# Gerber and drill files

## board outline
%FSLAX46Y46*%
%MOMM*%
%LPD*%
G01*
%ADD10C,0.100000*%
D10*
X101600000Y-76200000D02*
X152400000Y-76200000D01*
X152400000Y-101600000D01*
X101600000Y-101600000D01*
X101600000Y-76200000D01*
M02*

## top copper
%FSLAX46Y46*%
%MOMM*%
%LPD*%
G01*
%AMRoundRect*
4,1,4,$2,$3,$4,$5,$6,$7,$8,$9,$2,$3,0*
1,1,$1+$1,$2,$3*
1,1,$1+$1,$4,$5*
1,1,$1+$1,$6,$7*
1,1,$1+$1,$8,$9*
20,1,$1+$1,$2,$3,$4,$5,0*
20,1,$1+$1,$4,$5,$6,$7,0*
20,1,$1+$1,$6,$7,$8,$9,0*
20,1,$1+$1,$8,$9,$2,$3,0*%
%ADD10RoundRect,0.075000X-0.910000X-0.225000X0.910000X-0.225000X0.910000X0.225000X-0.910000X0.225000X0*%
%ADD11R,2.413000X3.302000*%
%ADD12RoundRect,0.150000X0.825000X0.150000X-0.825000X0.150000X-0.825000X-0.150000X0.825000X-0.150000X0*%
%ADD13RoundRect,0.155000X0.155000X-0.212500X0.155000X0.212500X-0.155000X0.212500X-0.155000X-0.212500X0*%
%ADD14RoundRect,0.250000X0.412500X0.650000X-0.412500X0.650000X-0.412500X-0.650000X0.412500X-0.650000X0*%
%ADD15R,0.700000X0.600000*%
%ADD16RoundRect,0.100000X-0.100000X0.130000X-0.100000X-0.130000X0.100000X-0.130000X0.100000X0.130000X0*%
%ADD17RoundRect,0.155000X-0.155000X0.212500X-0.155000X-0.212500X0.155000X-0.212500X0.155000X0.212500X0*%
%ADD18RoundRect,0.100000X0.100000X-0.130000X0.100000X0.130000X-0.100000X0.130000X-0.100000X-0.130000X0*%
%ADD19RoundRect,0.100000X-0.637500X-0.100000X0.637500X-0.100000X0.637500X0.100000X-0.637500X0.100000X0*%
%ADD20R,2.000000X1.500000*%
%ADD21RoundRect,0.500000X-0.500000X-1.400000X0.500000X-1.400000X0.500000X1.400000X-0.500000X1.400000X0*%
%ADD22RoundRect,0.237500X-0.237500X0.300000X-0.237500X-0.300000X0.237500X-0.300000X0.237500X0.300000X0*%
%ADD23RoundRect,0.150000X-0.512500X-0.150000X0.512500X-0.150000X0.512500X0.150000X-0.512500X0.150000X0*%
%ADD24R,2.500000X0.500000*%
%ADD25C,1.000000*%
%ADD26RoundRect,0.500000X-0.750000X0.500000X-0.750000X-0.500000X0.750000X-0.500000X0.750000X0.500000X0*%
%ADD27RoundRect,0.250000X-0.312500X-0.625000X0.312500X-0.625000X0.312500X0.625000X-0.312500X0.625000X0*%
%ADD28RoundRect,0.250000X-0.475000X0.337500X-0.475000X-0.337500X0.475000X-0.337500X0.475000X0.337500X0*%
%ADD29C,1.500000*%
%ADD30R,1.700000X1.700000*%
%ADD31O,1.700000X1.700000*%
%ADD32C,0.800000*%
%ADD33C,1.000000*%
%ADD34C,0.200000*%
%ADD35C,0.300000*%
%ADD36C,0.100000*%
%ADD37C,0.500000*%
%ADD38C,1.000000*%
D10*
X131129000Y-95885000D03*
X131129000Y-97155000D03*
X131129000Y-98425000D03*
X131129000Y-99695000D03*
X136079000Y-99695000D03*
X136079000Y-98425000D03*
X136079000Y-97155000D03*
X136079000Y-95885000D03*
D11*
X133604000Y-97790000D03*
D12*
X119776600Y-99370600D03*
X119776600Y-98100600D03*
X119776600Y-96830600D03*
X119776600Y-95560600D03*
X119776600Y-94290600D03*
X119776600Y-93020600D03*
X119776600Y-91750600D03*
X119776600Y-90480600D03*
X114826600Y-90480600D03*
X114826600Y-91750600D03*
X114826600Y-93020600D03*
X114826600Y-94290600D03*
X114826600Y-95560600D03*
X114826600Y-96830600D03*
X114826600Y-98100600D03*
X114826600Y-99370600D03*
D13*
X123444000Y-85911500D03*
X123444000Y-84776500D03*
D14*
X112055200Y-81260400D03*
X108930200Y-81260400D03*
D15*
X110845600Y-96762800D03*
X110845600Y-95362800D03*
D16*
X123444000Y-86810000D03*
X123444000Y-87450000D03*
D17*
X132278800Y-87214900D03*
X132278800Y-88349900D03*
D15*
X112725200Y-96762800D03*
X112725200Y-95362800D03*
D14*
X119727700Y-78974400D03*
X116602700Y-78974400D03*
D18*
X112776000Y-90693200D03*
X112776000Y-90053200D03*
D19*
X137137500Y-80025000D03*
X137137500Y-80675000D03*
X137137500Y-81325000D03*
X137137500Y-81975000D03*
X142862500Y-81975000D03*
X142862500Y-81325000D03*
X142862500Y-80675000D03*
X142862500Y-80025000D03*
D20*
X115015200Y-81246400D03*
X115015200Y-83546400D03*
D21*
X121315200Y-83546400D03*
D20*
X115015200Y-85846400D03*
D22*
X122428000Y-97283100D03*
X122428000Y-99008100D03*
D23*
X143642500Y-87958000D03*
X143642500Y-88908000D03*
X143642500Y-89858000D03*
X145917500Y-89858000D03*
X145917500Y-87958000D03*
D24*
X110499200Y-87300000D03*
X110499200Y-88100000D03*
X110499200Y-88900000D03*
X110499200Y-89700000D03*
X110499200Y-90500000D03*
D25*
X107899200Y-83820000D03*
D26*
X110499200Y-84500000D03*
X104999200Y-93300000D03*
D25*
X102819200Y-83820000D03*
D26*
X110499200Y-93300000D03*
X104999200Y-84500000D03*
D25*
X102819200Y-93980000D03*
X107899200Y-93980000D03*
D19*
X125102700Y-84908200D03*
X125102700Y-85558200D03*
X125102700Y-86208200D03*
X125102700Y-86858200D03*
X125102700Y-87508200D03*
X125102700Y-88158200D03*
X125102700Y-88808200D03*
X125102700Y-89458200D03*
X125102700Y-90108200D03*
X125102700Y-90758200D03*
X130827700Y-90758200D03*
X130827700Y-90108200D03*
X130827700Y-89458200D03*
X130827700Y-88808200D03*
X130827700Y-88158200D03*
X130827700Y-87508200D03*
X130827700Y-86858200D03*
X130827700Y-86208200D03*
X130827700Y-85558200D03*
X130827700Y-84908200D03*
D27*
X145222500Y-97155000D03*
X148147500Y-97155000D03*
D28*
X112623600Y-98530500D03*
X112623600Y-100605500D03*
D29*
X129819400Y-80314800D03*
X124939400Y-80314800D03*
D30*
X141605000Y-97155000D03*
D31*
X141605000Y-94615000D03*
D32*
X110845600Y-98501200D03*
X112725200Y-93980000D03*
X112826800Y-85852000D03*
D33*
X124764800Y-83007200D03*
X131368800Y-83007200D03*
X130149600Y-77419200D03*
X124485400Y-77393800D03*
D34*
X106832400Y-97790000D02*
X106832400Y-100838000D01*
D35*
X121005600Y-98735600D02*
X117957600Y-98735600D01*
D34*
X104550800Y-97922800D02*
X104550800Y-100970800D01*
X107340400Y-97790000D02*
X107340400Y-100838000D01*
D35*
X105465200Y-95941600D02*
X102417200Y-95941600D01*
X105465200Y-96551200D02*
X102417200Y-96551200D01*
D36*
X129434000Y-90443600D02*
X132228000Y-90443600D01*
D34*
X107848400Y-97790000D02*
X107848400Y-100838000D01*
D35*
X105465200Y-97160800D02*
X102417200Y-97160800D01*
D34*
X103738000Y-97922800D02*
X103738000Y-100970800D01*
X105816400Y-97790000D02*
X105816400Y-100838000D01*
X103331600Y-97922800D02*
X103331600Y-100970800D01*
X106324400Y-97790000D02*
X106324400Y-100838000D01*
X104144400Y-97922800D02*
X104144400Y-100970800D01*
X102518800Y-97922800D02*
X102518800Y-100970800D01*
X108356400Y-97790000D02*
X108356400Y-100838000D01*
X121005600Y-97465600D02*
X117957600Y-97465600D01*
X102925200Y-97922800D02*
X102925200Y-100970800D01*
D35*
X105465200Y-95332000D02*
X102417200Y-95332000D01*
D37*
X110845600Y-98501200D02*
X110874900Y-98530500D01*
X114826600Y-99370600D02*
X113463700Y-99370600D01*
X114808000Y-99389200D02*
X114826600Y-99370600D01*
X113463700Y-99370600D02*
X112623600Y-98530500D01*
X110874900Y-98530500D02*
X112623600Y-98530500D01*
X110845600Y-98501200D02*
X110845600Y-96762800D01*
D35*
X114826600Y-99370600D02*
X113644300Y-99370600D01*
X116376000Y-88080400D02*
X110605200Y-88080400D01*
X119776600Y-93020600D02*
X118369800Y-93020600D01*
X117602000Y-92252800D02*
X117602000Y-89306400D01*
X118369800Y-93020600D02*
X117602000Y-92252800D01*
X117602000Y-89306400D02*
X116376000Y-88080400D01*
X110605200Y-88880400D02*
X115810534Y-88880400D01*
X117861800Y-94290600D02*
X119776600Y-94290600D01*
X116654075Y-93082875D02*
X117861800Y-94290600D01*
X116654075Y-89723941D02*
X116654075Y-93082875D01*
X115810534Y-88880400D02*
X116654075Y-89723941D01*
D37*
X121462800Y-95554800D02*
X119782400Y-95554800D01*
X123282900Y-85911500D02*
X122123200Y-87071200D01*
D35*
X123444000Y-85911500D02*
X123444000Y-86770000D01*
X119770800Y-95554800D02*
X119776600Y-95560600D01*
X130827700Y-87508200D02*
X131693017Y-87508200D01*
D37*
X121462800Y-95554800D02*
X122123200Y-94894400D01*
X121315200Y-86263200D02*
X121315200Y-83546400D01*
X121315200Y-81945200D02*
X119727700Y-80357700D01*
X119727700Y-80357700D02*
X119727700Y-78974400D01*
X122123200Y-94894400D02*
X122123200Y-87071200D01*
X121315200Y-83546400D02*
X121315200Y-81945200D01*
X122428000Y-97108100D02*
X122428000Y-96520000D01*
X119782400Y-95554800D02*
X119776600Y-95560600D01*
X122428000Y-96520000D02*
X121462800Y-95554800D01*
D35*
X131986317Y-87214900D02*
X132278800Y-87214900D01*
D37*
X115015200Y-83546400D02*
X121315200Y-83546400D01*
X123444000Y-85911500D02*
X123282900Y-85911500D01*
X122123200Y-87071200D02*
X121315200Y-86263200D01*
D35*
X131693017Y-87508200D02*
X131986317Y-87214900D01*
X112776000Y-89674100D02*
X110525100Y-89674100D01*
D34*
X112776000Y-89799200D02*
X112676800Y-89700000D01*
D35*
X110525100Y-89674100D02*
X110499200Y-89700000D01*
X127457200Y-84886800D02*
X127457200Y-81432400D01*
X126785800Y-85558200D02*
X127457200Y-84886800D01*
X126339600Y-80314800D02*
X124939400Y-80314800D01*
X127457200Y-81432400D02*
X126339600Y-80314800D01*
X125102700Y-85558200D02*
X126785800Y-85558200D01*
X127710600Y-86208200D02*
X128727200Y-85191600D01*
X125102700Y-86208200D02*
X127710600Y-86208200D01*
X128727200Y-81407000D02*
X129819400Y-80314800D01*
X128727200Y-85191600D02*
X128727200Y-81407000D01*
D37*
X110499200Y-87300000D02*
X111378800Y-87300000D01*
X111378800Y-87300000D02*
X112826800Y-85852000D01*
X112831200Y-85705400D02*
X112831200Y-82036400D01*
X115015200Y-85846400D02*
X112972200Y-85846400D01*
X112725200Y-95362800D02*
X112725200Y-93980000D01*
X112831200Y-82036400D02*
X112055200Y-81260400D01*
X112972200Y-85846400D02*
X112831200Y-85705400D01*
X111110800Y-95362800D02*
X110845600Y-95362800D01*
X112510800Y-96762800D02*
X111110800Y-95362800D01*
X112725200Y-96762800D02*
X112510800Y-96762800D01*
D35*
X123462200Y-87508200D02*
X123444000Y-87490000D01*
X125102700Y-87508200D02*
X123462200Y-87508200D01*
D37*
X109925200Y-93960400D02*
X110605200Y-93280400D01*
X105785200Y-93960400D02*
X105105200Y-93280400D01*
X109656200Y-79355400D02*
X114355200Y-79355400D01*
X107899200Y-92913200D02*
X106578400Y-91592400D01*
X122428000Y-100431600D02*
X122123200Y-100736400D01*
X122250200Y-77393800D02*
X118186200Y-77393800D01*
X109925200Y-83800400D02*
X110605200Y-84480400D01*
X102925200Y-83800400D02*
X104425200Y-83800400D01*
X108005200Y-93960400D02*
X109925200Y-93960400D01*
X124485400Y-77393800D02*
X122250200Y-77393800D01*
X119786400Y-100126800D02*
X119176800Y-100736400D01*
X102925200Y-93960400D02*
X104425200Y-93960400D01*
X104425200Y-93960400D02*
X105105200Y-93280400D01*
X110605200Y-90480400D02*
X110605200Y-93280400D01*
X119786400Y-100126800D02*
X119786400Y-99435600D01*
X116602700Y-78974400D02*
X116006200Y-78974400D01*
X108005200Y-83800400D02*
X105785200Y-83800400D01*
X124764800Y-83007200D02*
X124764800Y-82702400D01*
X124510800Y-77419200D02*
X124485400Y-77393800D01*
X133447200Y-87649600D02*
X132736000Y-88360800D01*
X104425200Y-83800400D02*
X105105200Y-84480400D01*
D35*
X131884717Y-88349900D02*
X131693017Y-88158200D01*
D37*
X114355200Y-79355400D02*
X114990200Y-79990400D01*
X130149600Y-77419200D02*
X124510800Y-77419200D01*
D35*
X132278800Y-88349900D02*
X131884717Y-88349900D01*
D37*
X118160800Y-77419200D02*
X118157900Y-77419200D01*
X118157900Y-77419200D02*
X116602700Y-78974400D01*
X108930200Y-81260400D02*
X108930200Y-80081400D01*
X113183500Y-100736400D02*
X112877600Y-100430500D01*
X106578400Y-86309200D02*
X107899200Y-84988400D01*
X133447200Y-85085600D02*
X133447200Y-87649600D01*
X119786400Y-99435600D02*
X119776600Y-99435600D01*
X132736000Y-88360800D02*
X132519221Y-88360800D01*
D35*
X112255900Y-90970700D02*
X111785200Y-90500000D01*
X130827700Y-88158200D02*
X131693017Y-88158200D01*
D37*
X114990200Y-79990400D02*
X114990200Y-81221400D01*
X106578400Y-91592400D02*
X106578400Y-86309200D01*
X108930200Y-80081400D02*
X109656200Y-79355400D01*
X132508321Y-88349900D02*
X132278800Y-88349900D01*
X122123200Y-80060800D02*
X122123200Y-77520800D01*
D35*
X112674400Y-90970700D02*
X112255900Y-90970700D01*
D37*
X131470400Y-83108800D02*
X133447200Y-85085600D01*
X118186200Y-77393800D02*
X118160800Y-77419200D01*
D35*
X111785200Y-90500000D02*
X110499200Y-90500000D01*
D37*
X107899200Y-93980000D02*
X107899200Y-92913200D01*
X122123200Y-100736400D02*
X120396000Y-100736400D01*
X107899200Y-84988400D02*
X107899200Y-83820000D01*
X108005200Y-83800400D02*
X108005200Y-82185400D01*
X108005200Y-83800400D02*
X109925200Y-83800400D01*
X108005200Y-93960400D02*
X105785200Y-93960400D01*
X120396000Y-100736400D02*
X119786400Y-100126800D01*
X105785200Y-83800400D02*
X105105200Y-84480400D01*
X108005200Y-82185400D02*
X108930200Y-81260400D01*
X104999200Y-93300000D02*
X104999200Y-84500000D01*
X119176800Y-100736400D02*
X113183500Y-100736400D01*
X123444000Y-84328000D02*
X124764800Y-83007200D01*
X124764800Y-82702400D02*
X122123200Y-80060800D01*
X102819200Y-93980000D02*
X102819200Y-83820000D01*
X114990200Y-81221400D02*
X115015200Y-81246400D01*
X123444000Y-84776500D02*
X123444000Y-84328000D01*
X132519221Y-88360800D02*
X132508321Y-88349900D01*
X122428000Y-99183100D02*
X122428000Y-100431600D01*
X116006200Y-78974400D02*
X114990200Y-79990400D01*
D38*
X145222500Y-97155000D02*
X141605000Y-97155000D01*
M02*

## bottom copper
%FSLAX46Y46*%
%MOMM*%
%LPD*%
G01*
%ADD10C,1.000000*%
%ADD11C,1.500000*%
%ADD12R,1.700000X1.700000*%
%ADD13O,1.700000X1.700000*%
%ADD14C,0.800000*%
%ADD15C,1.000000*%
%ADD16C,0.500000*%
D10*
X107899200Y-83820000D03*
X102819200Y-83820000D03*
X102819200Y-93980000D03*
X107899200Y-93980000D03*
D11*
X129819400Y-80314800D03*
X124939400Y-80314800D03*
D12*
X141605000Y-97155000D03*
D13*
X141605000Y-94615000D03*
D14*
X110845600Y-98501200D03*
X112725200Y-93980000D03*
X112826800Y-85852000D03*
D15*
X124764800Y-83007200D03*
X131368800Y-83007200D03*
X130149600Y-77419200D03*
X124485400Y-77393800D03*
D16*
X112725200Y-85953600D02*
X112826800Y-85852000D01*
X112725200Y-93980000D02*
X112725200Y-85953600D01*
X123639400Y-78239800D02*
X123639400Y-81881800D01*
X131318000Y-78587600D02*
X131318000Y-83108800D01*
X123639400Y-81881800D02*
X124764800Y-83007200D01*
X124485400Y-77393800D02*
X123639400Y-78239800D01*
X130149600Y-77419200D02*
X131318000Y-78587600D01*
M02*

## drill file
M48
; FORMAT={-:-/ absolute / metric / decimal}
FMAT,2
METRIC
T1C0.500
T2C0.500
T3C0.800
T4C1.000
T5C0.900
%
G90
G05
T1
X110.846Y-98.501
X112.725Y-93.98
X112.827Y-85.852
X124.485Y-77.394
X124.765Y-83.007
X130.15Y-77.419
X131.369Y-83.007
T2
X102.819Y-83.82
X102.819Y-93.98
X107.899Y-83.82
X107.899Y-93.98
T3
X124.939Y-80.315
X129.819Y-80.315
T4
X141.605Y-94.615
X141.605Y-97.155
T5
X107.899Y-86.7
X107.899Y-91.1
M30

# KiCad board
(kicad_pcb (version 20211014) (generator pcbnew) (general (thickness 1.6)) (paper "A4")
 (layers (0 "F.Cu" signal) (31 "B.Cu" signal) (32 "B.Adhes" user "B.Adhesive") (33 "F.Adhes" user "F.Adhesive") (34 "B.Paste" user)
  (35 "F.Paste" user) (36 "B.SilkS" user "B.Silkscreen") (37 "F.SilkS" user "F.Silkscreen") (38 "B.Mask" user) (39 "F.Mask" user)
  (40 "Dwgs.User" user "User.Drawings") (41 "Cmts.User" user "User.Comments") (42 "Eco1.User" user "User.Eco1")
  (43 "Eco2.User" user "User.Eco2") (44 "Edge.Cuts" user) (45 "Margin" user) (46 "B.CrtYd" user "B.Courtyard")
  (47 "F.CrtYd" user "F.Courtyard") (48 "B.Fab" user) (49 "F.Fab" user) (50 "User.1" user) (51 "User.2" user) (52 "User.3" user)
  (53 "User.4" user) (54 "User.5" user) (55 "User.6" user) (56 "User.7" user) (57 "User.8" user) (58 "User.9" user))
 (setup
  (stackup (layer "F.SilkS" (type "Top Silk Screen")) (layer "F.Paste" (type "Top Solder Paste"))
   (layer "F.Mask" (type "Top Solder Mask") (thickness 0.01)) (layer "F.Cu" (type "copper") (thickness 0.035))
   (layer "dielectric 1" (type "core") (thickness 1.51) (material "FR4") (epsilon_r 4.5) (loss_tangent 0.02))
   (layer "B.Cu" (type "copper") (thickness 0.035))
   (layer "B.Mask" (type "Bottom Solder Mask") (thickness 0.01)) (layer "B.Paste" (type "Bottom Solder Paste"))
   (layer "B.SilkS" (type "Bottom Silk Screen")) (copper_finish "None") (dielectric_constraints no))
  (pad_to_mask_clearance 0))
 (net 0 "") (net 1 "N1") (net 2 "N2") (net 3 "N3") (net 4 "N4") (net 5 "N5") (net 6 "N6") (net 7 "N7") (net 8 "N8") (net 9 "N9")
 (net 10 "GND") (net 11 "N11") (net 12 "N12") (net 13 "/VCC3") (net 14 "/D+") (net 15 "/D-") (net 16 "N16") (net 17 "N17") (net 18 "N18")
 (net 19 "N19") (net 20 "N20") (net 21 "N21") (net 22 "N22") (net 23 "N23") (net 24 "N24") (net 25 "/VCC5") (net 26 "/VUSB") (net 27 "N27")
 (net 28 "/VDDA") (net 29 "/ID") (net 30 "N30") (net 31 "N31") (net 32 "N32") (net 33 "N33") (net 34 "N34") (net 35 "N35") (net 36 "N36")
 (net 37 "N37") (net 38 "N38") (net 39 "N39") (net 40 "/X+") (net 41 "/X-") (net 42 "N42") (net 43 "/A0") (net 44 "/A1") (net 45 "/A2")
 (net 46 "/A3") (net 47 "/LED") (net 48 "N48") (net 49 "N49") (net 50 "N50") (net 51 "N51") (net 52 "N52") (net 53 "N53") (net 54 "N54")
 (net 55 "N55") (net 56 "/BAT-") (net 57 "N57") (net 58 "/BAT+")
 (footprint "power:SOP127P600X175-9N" (layer "F.Cu") (at 133.604 97.79)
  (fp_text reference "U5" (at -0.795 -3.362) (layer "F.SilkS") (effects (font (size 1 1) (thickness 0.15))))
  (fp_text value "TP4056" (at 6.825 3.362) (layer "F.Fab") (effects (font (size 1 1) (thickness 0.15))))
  (pad "1" smd roundrect locked (at -2.475 -1.905) (size 1.97 0.6) (layers "F.Cu" "F.Paste" "F.Mask") (roundrect_rratio 0.125) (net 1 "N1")
   (solder_mask_margin 0.102))
  (pad "2" smd roundrect locked (at -2.475 -0.635) (size 1.97 0.6) (layers "F.Cu" "F.Paste" "F.Mask") (roundrect_rratio 0.125) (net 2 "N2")
   (solder_mask_margin 0.102))
  (pad "3" smd roundrect locked (at -2.475 0.635) (size 1.97 0.6) (layers "F.Cu" "F.Paste" "F.Mask") (roundrect_rratio 0.125) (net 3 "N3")
   (solder_mask_margin 0.102))
  (pad "4" smd roundrect locked (at -2.475 1.905) (size 1.97 0.6) (layers "F.Cu" "F.Paste" "F.Mask") (roundrect_rratio 0.125) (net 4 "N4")
   (solder_mask_margin 0.102))
  (pad "5" smd roundrect locked (at 2.475 1.905) (size 1.97 0.6) (layers "F.Cu" "F.Paste" "F.Mask") (roundrect_rratio 0.125) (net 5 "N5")
   (solder_mask_margin 0.102))
  (pad "6" smd roundrect locked (at 2.475 0.635) (size 1.97 0.6) (layers "F.Cu" "F.Paste" "F.Mask") (roundrect_rratio 0.125) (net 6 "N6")
   (solder_mask_margin 0.102))
  (pad "7" smd roundrect locked (at 2.475 -0.635) (size 1.97 0.6) (layers "F.Cu" "F.Paste" "F.Mask") (roundrect_rratio 0.125) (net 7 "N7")
   (solder_mask_margin 0.102))
  (pad "8" smd roundrect locked (at 2.475 -1.905) (size 1.97 0.6) (layers "F.Cu" "F.Paste" "F.Mask") (roundrect_rratio 0.125) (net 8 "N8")
   (solder_mask_margin 0.102))
  (pad "9" smd rect locked (at 0 0) (size 2.413 3.302) (layers "F.Cu" "F.Mask") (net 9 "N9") (solder_mask_margin 0.102)))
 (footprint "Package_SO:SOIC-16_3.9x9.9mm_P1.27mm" (layer "F.Cu") (at 117.3016 94.9256 180) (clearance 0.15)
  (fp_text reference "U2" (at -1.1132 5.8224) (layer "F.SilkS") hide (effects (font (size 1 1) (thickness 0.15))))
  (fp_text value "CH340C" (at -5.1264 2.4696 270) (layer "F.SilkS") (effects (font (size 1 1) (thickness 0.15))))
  (pad "1" smd roundrect (at -2.475 -4.445 180) (size 1.95 0.6) (layers "F.Cu" "F.Paste" "F.Mask") (roundrect_rratio 0.25) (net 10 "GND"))
  (pad "2" smd roundrect (at -2.475 -3.175 180) (size 1.95 0.6) (layers "F.Cu" "F.Paste" "F.Mask") (roundrect_rratio 0.25) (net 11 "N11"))
  (pad "3" smd roundrect (at -2.475 -1.905 180) (size 1.95 0.6) (layers "F.Cu" "F.Paste" "F.Mask") (roundrect_rratio 0.25) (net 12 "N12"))
  (pad "4" smd roundrect (at -2.475 -0.635 180) (size 1.95 0.6) (layers "F.Cu" "F.Paste" "F.Mask") (roundrect_rratio 0.25) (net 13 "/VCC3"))
  (pad "5" smd roundrect (at -2.475 0.635 180) (size 1.95 0.6) (layers "F.Cu" "F.Paste" "F.Mask") (roundrect_rratio 0.25) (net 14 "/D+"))
  (pad "6" smd roundrect (at -2.475 1.905 180) (size 1.95 0.6) (layers "F.Cu" "F.Paste" "F.Mask") (roundrect_rratio 0.25) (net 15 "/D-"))
  (pad "7" smd roundrect (at -2.475 3.175 180) (size 1.95 0.6) (layers "F.Cu" "F.Paste" "F.Mask") (roundrect_rratio 0.25) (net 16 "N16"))
  (pad "8" smd roundrect (at -2.475 4.445 180) (size 1.95 0.6) (layers "F.Cu" "F.Paste" "F.Mask") (roundrect_rratio 0.25) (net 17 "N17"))
  (pad "9" smd roundrect (at 2.475 4.445 180) (size 1.95 0.6) (layers "F.Cu" "F.Paste" "F.Mask") (roundrect_rratio 0.25) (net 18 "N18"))
  (pad "10" smd roundrect (at 2.475 3.175 180) (size 1.95 0.6) (layers "F.Cu" "F.Paste" "F.Mask") (roundrect_rratio 0.25) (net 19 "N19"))
  (pad "11" smd roundrect (at 2.475 1.905 180) (size 1.95 0.6) (layers "F.Cu" "F.Paste" "F.Mask") (roundrect_rratio 0.25) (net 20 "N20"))
  (pad "12" smd roundrect (at 2.475 0.635 180) (size 1.95 0.6) (layers "F.Cu" "F.Paste" "F.Mask") (roundrect_rratio 0.25) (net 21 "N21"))
  (pad "13" smd roundrect (at 2.475 -0.635 180) (size 1.95 0.6) (layers "F.Cu" "F.Paste" "F.Mask") (roundrect_rratio 0.25) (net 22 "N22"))
  (pad "14" smd roundrect (at 2.475 -1.905 180) (size 1.95 0.6) (layers "F.Cu" "F.Paste" "F.Mask") (roundrect_rratio 0.25) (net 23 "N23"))
  (pad "15" smd roundrect (at 2.475 -3.175 180) (size 1.95 0.6) (layers "F.Cu" "F.Paste" "F.Mask") (roundrect_rratio 0.25) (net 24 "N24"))
  (pad "16" smd roundrect (at 2.475 -4.445 180) (size 1.95 0.6) (layers "F.Cu" "F.Paste" "F.Mask") (roundrect_rratio 0.25) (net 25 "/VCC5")))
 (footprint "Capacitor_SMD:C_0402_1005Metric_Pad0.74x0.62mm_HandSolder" (layer "F.Cu") (at 123.444 85.344 90)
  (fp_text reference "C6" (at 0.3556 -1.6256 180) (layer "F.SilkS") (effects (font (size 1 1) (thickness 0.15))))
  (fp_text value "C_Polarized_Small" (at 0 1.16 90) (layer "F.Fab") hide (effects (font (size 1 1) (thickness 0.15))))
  (pad "1" smd roundrect (at -0.5675 0 90) (size 0.735 0.62) (layers "F.Cu" "F.Paste" "F.Mask") (roundrect_rratio 0.25) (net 13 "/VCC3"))
  (pad "2" smd roundrect (at 0.5675 0 90) (size 0.735 0.62) (layers "F.Cu" "F.Paste" "F.Mask") (roundrect_rratio 0.25) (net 10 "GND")))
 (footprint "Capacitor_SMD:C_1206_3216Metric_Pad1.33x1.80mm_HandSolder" (layer "F.Cu") (at 110.4927 81.2604 180)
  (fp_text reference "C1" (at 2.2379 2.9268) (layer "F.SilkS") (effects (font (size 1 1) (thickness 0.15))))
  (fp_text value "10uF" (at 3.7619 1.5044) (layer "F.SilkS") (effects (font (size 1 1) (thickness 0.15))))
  (pad "1" smd roundrect (at -1.5625 0 180) (size 1.325 1.8) (layers "F.Cu" "F.Paste" "F.Mask") (roundrect_rratio 0.188679) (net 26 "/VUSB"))
  (pad "2" smd roundrect (at 1.5625 0 180) (size 1.325 1.8) (layers "F.Cu" "F.Paste" "F.Mask") (roundrect_rratio 0.188679) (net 10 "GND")))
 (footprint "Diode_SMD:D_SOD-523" (layer "F.Cu") (at 110.8456 96.0628 90)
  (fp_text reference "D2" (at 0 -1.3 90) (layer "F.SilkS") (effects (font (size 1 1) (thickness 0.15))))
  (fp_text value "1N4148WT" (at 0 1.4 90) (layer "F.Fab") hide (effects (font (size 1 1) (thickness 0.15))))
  (pad "1" smd rect (at -0.7 0 270) (size 0.6 0.7) (layers "F.Cu" "F.Paste" "F.Mask") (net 25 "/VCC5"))
  (pad "2" smd rect (at 0.7 0 270) (size 0.6 0.7) (layers "F.Cu" "F.Paste" "F.Mask") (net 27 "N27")))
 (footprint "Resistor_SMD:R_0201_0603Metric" (layer "F.Cu") (at 123.444 87.13 -90)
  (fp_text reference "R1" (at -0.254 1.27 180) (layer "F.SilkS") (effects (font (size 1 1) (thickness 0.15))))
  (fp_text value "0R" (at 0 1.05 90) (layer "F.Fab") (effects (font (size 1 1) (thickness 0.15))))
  (pad "" smd roundrect (at -0.345 0 270) (size 0.318 0.36) (layers "F.Paste") (roundrect_rratio 0.25))
  (pad "" smd roundrect (at 0.345 0 270) (size 0.318 0.36) (layers "F.Paste") (roundrect_rratio 0.25))
  (pad "1" smd roundrect (at -0.32 0 270) (size 0.46 0.4) (layers "F.Cu" "F.Mask") (roundrect_rratio 0.25) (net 13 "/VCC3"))
  (pad "2" smd roundrect (at 0.32 0 270) (size 0.46 0.4) (layers "F.Cu" "F.Mask") (roundrect_rratio 0.25) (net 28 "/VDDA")))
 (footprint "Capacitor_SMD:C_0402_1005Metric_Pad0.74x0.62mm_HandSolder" (layer "F.Cu") (at 132.2788 87.7824 -90)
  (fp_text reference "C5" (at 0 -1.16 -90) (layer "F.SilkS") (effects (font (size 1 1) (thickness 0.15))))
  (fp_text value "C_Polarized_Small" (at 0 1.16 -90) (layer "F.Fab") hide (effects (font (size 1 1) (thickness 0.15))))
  (pad "1" smd roundrect (at -0.5675 0 270) (size 0.735 0.62) (layers "F.Cu" "F.Paste" "F.Mask") (roundrect_rratio 0.25) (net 13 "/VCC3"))
  (pad "2" smd roundrect (at 0.5675 0 270) (size 0.735 0.62) (layers "F.Cu" "F.Paste" "F.Mask") (roundrect_rratio 0.25) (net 10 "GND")))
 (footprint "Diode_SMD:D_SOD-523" (layer "F.Cu") (at 112.7252 96.0628 90)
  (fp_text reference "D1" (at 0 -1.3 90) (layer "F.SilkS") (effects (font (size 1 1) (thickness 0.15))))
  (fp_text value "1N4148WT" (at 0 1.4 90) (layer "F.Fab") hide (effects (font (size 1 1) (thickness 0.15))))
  (pad "1" smd rect (at -0.7 0 270) (size 0.6 0.7) (layers "F.Cu" "F.Paste" "F.Mask") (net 27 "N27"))
  (pad "2" smd rect (at 0.7 0 270) (size 0.6 0.7) (layers "F.Cu" "F.Paste" "F.Mask") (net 26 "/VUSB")))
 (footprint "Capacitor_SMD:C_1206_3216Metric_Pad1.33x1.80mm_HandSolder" (layer "F.Cu") (at 118.1652 78.9744 180)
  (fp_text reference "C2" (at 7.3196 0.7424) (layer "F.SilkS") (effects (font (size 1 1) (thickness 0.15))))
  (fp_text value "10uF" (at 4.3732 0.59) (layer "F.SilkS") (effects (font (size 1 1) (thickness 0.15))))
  (pad "1" smd roundrect (at -1.5625 0 180) (size 1.325 1.8) (layers "F.Cu" "F.Paste" "F.Mask") (roundrect_rratio 0.188679) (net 13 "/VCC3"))
  (pad "2" smd roundrect (at 1.5625 0 180) (size 1.325 1.8) (layers "F.Cu" "F.Paste" "F.Mask") (roundrect_rratio 0.188679) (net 10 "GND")))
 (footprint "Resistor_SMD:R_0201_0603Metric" (layer "F.Cu") (at 112.776 90.3732 90)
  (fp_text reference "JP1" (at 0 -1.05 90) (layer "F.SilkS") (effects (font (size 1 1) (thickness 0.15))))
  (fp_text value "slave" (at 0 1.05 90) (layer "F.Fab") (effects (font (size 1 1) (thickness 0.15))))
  (pad "" smd roundrect (at -0.345 0 90) (size 0.318 0.36) (layers "F.Paste") (roundrect_rratio 0.25))
  (pad "" smd roundrect (at 0.345 0 90) (size 0.318 0.36) (layers "F.Paste") (roundrect_rratio 0.25))
  (pad "1" smd roundrect (at -0.32 0 90) (size 0.46 0.4) (layers "F.Cu" "F.Mask") (roundrect_rratio 0.25) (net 10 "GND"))
  (pad "2" smd roundrect (at 0.32 0 90) (size 0.46 0.4) (layers "F.Cu" "F.Mask") (roundrect_rratio 0.25) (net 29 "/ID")))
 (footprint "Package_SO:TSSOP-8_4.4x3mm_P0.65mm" (layer "F.Cu") (at 140 81)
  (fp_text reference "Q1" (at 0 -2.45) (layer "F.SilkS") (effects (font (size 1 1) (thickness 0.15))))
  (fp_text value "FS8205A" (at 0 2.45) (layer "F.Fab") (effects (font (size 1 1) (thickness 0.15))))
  (pad "1" smd roundrect (at -2.8625 -0.975) (size 1.475 0.4) (layers "F.Cu" "F.Paste" "F.Mask") (roundrect_rratio 0.25) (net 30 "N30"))
  (pad "2" smd roundrect (at -2.8625 -0.325) (size 1.475 0.4) (layers "F.Cu" "F.Paste" "F.Mask") (roundrect_rratio 0.25) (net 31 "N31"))
  (pad "3" smd roundrect (at -2.8625 0.325) (size 1.475 0.4) (layers "F.Cu" "F.Paste" "F.Mask") (roundrect_rratio 0.25) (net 31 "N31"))
  (pad "4" smd roundrect (at -2.8625 0.975) (size 1.475 0.4) (layers "F.Cu" "F.Paste" "F.Mask") (roundrect_rratio 0.25) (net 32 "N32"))
  (pad "5" smd roundrect (at 2.8625 0.975) (size 1.475 0.4) (layers "F.Cu" "F.Paste" "F.Mask") (roundrect_rratio 0.25) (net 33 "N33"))
  (pad "6" smd roundrect (at 2.8625 0.325) (size 1.475 0.4) (layers "F.Cu" "F.Paste" "F.Mask") (roundrect_rratio 0.25) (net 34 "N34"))
  (pad "7" smd roundrect (at 2.8625 -0.325) (size 1.475 0.4) (layers "F.Cu" "F.Paste" "F.Mask") (roundrect_rratio 0.25) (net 34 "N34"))
  (pad "8" smd roundrect (at 2.8625 -0.975) (size 1.475 0.4) (layers "F.Cu" "F.Paste" "F.Mask") (roundrect_rratio 0.25) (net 30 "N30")))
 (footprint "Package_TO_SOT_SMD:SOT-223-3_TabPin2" (layer "F.Cu") (at 118.1652 83.5464)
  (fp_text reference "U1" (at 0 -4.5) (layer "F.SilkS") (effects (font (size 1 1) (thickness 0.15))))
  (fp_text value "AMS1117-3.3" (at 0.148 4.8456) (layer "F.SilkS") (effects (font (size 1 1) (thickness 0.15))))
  (pad "1" smd rect (at -3.15 -2.3) (size 2 1.5) (layers "F.Cu" "F.Paste" "F.Mask") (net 10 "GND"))
  (pad "2" smd rect (at -3.15 0) (size 2 1.5) (layers "F.Cu" "F.Paste" "F.Mask") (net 13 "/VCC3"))
  (pad "2" smd roundrect (at 3.15 0) (size 2 3.8) (layers "F.Cu" "F.Paste" "F.Mask") (roundrect_rratio 0.25) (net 13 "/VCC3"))
  (pad "3" smd rect (at -3.15 2.3) (size 2 1.5) (layers "F.Cu" "F.Paste" "F.Mask") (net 26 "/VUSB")))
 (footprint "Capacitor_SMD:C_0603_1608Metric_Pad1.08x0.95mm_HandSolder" (layer "F.Cu") (at 122.428 98.1456 -90)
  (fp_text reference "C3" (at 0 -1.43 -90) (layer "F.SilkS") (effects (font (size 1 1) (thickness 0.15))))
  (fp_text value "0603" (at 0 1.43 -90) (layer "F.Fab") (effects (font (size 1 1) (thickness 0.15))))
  (pad "1" smd roundrect (at -0.8625 0 270) (size 1.075 0.95) (layers "F.Cu" "F.Paste" "F.Mask") (roundrect_rratio 0.25) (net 13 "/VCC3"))
  (pad "2" smd roundrect (at 0.8625 0 270) (size 1.075 0.95) (layers "F.Cu" "F.Paste" "F.Mask") (roundrect_rratio 0.25) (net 10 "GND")))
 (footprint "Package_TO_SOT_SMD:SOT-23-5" (layer "F.Cu") (at 144.78 88.908)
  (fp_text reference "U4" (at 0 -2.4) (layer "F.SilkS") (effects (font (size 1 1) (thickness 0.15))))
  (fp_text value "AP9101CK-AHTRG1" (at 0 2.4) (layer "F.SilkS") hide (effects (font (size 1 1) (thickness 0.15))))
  (pad "1" smd roundrect (at -1.1375 -0.95) (size 1.325 0.6) (layers "F.Cu" "F.Paste" "F.Mask") (roundrect_rratio 0.25) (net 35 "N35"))
  (pad "2" smd roundrect (at -1.1375 0) (size 1.325 0.6) (layers "F.Cu" "F.Paste" "F.Mask") (roundrect_rratio 0.25) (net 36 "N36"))
  (pad "3" smd roundrect (at -1.1375 0.95) (size 1.325 0.6) (layers "F.Cu" "F.Paste" "F.Mask") (roundrect_rratio 0.25) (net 10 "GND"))
  (pad "4" smd roundrect (at 1.1375 0.95) (size 1.325 0.6) (layers "F.Cu" "F.Paste" "F.Mask") (roundrect_rratio 0.25) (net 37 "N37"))
  (pad "5" smd roundrect (at 1.1375 -0.95) (size 1.325 0.6) (layers "F.Cu" "F.Paste" "F.Mask") (roundrect_rratio 0.25) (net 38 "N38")))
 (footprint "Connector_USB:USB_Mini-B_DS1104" (layer "F.Cu") (at 107.8992 88.9 -90)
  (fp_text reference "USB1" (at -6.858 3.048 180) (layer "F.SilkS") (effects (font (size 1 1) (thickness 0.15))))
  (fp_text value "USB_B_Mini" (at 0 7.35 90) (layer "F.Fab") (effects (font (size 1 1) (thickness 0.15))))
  (pad "" np_thru_hole circle (at 2.2 0 270) (size 0.9 0.9) (drill 0.9) (layers *.Cu *.Mask))
  (pad "" np_thru_hole circle (at -2.2 0 270) (size 0.9 0.9) (drill 0.9) (layers *.Cu *.Mask))
  (pad "1" smd rect (at -1.6 -2.6 270) (size 0.5 2.5) (layers "F.Cu" "F.Paste" "F.Mask") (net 26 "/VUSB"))
  (pad "2" smd rect (at -0.8 -2.6 270) (size 0.5 2.5) (layers "F.Cu" "F.Paste" "F.Mask") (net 15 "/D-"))
  (pad "3" smd rect (at 0 -2.6 270) (size 0.5 2.5) (layers "F.Cu" "F.Paste" "F.Mask") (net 14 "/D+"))
  (pad "4" smd rect (at 0.8 -2.6 270) (size 0.5 2.5) (layers "F.Cu" "F.Paste" "F.Mask") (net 29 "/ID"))
  (pad "5" smd rect (at 1.6 -2.6 270) (size 0.5 2.5) (layers "F.Cu" "F.Paste" "F.Mask") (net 10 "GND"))
  (pad "6" thru_hole circle (at -5.08 0 270) (size 1 1) (drill 0.5) (layers *.Cu *.Mask) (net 10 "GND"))
  (pad "6" smd roundrect (at -4.4 -2.6 270) (size 2 2.5) (layers "F.Cu" "F.Paste" "F.Mask") (roundrect_rratio 0.25) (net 10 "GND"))
  (pad "6" smd roundrect (at 4.4 2.9 270) (size 2 2.5) (layers "F.Cu" "F.Paste" "F.Mask") (roundrect_rratio 0.25) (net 10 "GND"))
  (pad "6" thru_hole circle (at -5.08 5.08 270) (size 1 1) (drill 0.5) (layers *.Cu *.Mask) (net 10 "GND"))
  (pad "6" smd roundrect (at 4.4 -2.6 270) (size 2 2.5) (layers "F.Cu" "F.Paste" "F.Mask") (roundrect_rratio 0.25) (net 10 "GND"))
  (pad "6" smd roundrect (at -4.4 2.9 270) (size 2 2.5) (layers "F.Cu" "F.Paste" "F.Mask") (roundrect_rratio 0.25) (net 10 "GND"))
  (pad "6" thru_hole circle (at 5.08 5.08 270) (size 1 1) (drill 0.5) (layers *.Cu *.Mask) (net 10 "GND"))
  (pad "6" thru_hole circle (at 5.08 0 270) (size 1 1) (drill 0.5) (layers *.Cu *.Mask) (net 10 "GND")))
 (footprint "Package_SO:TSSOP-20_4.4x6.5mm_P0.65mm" (layer "F.Cu") (at 127.9652 87.8332)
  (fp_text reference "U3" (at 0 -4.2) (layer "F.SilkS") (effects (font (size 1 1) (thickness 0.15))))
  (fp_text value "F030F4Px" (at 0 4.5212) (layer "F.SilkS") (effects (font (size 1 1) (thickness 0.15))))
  (pad "1" smd roundrect (at -2.8625 -2.925) (size 1.475 0.4) (layers "F.Cu" "F.Paste" "F.Mask") (roundrect_rratio 0.25) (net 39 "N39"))
  (pad "2" smd roundrect (at -2.8625 -2.275) (size 1.475 0.4) (layers "F.Cu" "F.Paste" "F.Mask") (roundrect_rratio 0.25) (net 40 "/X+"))
  (pad "3" smd roundrect (at -2.8625 -1.625) (size 1.475 0.4) (layers "F.Cu" "F.Paste" "F.Mask") (roundrect_rratio 0.25) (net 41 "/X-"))
  (pad "4" smd roundrect (at -2.8625 -0.975) (size 1.475 0.4) (layers "F.Cu" "F.Paste" "F.Mask") (roundrect_rratio 0.25) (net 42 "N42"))
  (pad "5" smd roundrect (at -2.8625 -0.325) (size 1.475 0.4) (layers "F.Cu" "F.Paste" "F.Mask") (roundrect_rratio 0.25) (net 28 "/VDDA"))
  (pad "6" smd roundrect (at -2.8625 0.325) (size 1.475 0.4) (layers "F.Cu" "F.Paste" "F.Mask") (roundrect_rratio 0.25) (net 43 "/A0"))
  (pad "7" smd roundrect (at -2.8625 0.975) (size 1.475 0.4) (layers "F.Cu" "F.Paste" "F.Mask") (roundrect_rratio 0.25) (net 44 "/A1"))
  (pad "8" smd roundrect (at -2.8625 1.625) (size 1.475 0.4) (layers "F.Cu" "F.Paste" "F.Mask") (roundrect_rratio 0.25) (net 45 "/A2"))
  (pad "9" smd roundrect (at -2.8625 2.275) (size 1.475 0.4) (layers "F.Cu" "F.Paste" "F.Mask") (roundrect_rratio 0.25) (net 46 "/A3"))
  (pad "10" smd roundrect (at -2.8625 2.925) (size 1.475 0.4) (layers "F.Cu" "F.Paste" "F.Mask") (roundrect_rratio 0.25) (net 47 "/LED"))
  (pad "11" smd roundrect (at 2.8625 2.925) (size 1.475 0.4) (layers "F.Cu" "F.Paste" "F.Mask") (roundrect_rratio 0.25) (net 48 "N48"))
  (pad "12" smd roundrect (at 2.8625 2.275) (size 1.475 0.4) (layers "F.Cu" "F.Paste" "F.Mask") (roundrect_rratio 0.25) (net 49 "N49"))
  (pad "13" smd roundrect (at 2.8625 1.625) (size 1.475 0.4) (layers "F.Cu" "F.Paste" "F.Mask") (roundrect_rratio 0.25) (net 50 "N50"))
  (pad "14" smd roundrect (at 2.8625 0.975) (size 1.475 0.4) (layers "F.Cu" "F.Paste" "F.Mask") (roundrect_rratio 0.25) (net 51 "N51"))
  (pad "15" smd roundrect (at 2.8625 0.325) (size 1.475 0.4) (layers "F.Cu" "F.Paste" "F.Mask") (roundrect_rratio 0.25) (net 10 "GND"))
  (pad "16" smd roundrect (at 2.8625 -0.325) (size 1.475 0.4) (layers "F.Cu" "F.Paste" "F.Mask") (roundrect_rratio 0.25) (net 13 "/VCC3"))
  (pad "17" smd roundrect (at 2.8625 -0.975) (size 1.475 0.4) (layers "F.Cu" "F.Paste" "F.Mask") (roundrect_rratio 0.25) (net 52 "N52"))
  (pad "18" smd roundrect (at 2.8625 -1.625) (size 1.475 0.4) (layers "F.Cu" "F.Paste" "F.Mask") (roundrect_rratio 0.25) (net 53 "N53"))
  (pad "19" smd roundrect (at 2.8625 -2.275) (size 1.475 0.4) (layers "F.Cu" "F.Paste" "F.Mask") (roundrect_rratio 0.25) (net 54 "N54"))
  (pad "20" smd roundrect (at 2.8625 -2.925) (size 1.475 0.4) (layers "F.Cu" "F.Paste" "F.Mask") (roundrect_rratio 0.25) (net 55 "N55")))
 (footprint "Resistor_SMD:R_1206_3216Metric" (layer "F.Cu") (at 146.685 97.155)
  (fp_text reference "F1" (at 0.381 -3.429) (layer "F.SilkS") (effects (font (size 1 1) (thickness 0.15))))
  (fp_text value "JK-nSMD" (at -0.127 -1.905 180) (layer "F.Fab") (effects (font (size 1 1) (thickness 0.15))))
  (pad "1" smd roundrect (at -1.4625 0) (size 1.125 1.75) (layers "F.Cu" "F.Paste" "F.Mask") (roundrect_rratio 0.222222) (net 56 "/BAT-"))
  (pad "2" smd roundrect (at 1.4625 0) (size 1.125 1.75) (layers "F.Cu" "F.Paste" "F.Mask") (roundrect_rratio 0.222222) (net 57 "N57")))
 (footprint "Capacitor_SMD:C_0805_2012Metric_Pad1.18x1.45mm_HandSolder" (layer "F.Cu") (at 112.6236 99.568 -90)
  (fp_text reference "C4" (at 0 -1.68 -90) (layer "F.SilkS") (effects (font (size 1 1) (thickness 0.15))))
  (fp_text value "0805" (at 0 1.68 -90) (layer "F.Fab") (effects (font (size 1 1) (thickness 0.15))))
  (pad "1" smd roundrect (at -1.0375 0 270) (size 1.175 1.45) (layers "F.Cu" "F.Paste" "F.Mask") (roundrect_rratio 0.212766)
   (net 25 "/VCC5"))
  (pad "2" smd roundrect (at 1.0375 0 270) (size 1.175 1.45) (layers "F.Cu" "F.Paste" "F.Mask") (roundrect_rratio 0.212766) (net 10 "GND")))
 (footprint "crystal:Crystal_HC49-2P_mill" (layer "B.Cu") (at 129.8194 80.3148 180)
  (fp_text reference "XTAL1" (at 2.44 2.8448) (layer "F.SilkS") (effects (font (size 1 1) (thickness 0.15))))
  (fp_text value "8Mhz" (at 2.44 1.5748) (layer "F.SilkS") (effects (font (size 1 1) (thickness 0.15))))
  (pad "1" thru_hole circle (at 0 0 180) (size 1.5 1.5) (drill 0.8) (layers *.Cu *.Mask) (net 41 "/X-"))
  (pad "2" thru_hole circle (at 4.88 0 180) (size 1.5 1.5) (drill 0.8) (layers *.Cu *.Mask) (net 40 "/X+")))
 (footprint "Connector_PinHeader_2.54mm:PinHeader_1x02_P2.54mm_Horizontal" (layer "B.Cu") (at 141.605 97.155)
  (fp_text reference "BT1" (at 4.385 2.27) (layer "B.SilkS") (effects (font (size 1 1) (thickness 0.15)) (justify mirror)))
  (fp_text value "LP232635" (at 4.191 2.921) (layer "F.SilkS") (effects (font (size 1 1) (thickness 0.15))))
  (pad "1" thru_hole rect (at 0 0) (size 1.7 1.7) (drill 1) (layers *.Cu *.Mask) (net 56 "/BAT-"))
  (pad "2" thru_hole oval (at 0 -2.54) (size 1.7 1.7) (drill 1) (layers *.Cu *.Mask) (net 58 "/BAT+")))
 (gr_rect (start 101.6 76.2) (end 152.4 101.6) (layer "Edge.Cuts") (width 0.1) (fill none))
 (segment (start 106.8324 97.79) (end 106.8324 100.838) (width 0.2) (layer "F.Cu") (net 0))
 (segment (start 121.0056 98.7356) (end 117.9576 98.7356) (width 0.3) (layer "F.Cu") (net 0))
 (segment (start 104.5508 97.9228) (end 104.5508 100.9708) (width 0.2) (layer "F.Cu") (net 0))
 (segment (start 107.3404 97.79) (end 107.3404 100.838) (width 0.2) (layer "F.Cu") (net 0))
 (segment (start 105.4652 95.9416) (end 102.4172 95.9416) (width 0.3) (layer "F.Cu") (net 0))
 (segment (start 105.4652 96.5512) (end 102.4172 96.5512) (width 0.3) (layer "F.Cu") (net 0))
 (segment (start 129.434 90.4436) (end 132.228 90.4436) (width 0.1) (layer "F.Cu") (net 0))
 (segment (start 107.8484 97.79) (end 107.8484 100.838) (width 0.2) (layer "F.Cu") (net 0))
 (segment (start 105.4652 97.1608) (end 102.4172 97.1608) (width 0.3) (layer "F.Cu") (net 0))
 (segment (start 103.738 97.9228) (end 103.738 100.9708) (width 0.2) (layer "F.Cu") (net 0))
 (segment (start 105.8164 97.79) (end 105.8164 100.838) (width 0.2) (layer "F.Cu") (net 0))
 (segment (start 103.3316 97.9228) (end 103.3316 100.9708) (width 0.2) (layer "F.Cu") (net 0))
 (segment (start 106.3244 97.79) (end 106.3244 100.838) (width 0.2) (layer "F.Cu") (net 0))
 (segment (start 104.1444 97.9228) (end 104.1444 100.9708) (width 0.2) (layer "F.Cu") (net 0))
 (segment (start 102.5188 97.9228) (end 102.5188 100.9708) (width 0.2) (layer "F.Cu") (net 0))
 (segment (start 108.3564 97.79) (end 108.3564 100.838) (width 0.2) (layer "F.Cu") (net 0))
 (segment (start 121.0056 97.4656) (end 117.9576 97.4656) (width 0.2) (layer "F.Cu") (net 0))
 (segment (start 102.9252 97.9228) (end 102.9252 100.9708) (width 0.2) (layer "F.Cu") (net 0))
 (segment (start 105.4652 95.332) (end 102.4172 95.332) (width 0.3) (layer "F.Cu") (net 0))
 (segment (start 110.8456 98.5012) (end 110.8749 98.5305) (width 0.5) (layer "F.Cu") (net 25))
 (segment (start 114.8266 99.3706) (end 113.4637 99.3706) (width 0.5) (layer "F.Cu") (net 25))
 (segment (start 114.808 99.3892) (end 114.8266 99.3706) (width 0.5) (layer "F.Cu") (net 25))
 (segment (start 113.4637 99.3706) (end 112.6236 98.5305) (width 0.5) (layer "F.Cu") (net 25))
 (segment (start 110.8749 98.5305) (end 112.6236 98.5305) (width 0.5) (layer "F.Cu") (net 25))
 (segment (start 110.8456 98.5012) (end 110.8456 96.7628) (width 0.5) (layer "F.Cu") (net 25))
 (segment (start 114.8266 99.3706) (end 113.6443 99.3706) (width 0.3) (layer "F.Cu") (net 25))
 (via (at 110.8456 98.5012) (size 0.8) (drill 0.5) (layers "F.Cu" "B.Cu") (free) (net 25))
 (segment (start 116.376 88.0804) (end 110.6052 88.0804) (width 0.3) (layer "F.Cu") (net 15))
 (segment (start 119.7766 93.0206) (end 118.3698 93.0206) (width 0.3) (layer "F.Cu") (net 15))
 (segment (start 117.602 92.2528) (end 117.602 89.3064) (width 0.3) (layer "F.Cu") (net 15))
 (segment (start 118.3698 93.0206) (end 117.602 92.2528) (width 0.3) (layer "F.Cu") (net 15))
 (segment (start 117.602 89.3064) (end 116.376 88.0804) (width 0.3) (layer "F.Cu") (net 15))
 (segment (start 110.6052 88.8804) (end 115.810534 88.8804) (width 0.3) (layer "F.Cu") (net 14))
 (segment (start 117.8618 94.2906) (end 119.7766 94.2906) (width 0.3) (layer "F.Cu") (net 14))
 (segment (start 116.654075 93.082875) (end 117.8618 94.2906) (width 0.3) (layer "F.Cu") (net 14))
 (segment (start 116.654075 89.723941) (end 116.654075 93.082875) (width 0.3) (layer "F.Cu") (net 14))
 (segment (start 115.810534 88.8804) (end 116.654075 89.723941) (width 0.3) (layer "F.Cu") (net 14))
 (segment (start 121.4628 95.5548) (end 119.7824 95.5548) (width 0.5) (layer "F.Cu") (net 13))
 (segment (start 123.2829 85.9115) (end 122.1232 87.0712) (width 0.5) (layer "F.Cu") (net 13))
 (segment (start 123.444 85.9115) (end 123.444 86.77) (width 0.3) (layer "F.Cu") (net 13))
 (segment (start 119.7708 95.5548) (end 119.7766 95.5606) (width 0.3) (layer "F.Cu") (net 13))
 (segment (start 130.8277 87.5082) (end 131.693017 87.5082) (width 0.3) (layer "F.Cu") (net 13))
 (segment (start 121.4628 95.5548) (end 122.1232 94.8944) (width 0.5) (layer "F.Cu") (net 13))
 (segment (start 121.3152 86.2632) (end 121.3152 83.5464) (width 0.5) (layer "F.Cu") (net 13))
 (segment (start 121.3152 81.9452) (end 119.7277 80.3577) (width 0.5) (layer "F.Cu") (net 13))
 (segment (start 119.7277 80.3577) (end 119.7277 78.9744) (width 0.5) (layer "F.Cu") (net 13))
 (segment (start 122.1232 94.8944) (end 122.1232 87.0712) (width 0.5) (layer "F.Cu") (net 13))
 (segment (start 121.3152 83.5464) (end 121.3152 81.9452) (width 0.5) (layer "F.Cu") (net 13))
 (segment (start 122.428 97.1081) (end 122.428 96.52) (width 0.5) (layer "F.Cu") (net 13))
 (segment (start 119.7824 95.5548) (end 119.7766 95.5606) (width 0.5) (layer "F.Cu") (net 13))
 (segment (start 122.428 96.52) (end 121.4628 95.5548) (width 0.5) (layer "F.Cu") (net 13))
 (segment (start 131.986317 87.2149) (end 132.2788 87.2149) (width 0.3) (layer "F.Cu") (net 13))
 (segment (start 115.0152 83.5464) (end 121.3152 83.5464) (width 0.5) (layer "F.Cu") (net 13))
 (segment (start 123.444 85.9115) (end 123.2829 85.9115) (width 0.5) (layer "F.Cu") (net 13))
 (segment (start 122.1232 87.0712) (end 121.3152 86.2632) (width 0.5) (layer "F.Cu") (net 13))
 (segment (start 131.693017 87.5082) (end 131.986317 87.2149) (width 0.3) (layer "F.Cu") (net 13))
 (segment (start 112.776 89.6741) (end 110.5251 89.6741) (width 0.3) (layer "F.Cu") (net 29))
 (segment (start 112.776 89.7992) (end 112.6768 89.7) (width 0.2) (layer "F.Cu") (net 29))
 (segment (start 110.5251 89.6741) (end 110.4992 89.7) (width 0.3) (layer "F.Cu") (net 29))
 (segment (start 127.4572 84.8868) (end 127.4572 81.4324) (width 0.3) (layer "F.Cu") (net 40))
 (segment (start 126.7858 85.5582) (end 127.4572 84.8868) (width 0.3) (layer "F.Cu") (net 40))
 (segment (start 126.3396 80.3148) (end 124.9394 80.3148) (width 0.3) (layer "F.Cu") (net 40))
 (segment (start 127.4572 81.4324) (end 126.3396 80.3148) (width 0.3) (layer "F.Cu") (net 40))
 (segment (start 125.1027 85.5582) (end 126.7858 85.5582) (width 0.3) (layer "F.Cu") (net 40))
 (segment (start 127.7106 86.2082) (end 128.7272 85.1916) (width 0.3) (layer "F.Cu") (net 41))
 (segment (start 125.1027 86.2082) (end 127.7106 86.2082) (width 0.3) (layer "F.Cu") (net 41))
 (segment (start 128.7272 81.407) (end 129.8194 80.3148) (width 0.3) (layer "F.Cu") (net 41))
 (segment (start 128.7272 85.1916) (end 128.7272 81.407) (width 0.3) (layer "F.Cu") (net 41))
 (segment (start 110.4992 87.3) (end 111.3788 87.3) (width 0.5) (layer "F.Cu") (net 26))
 (segment (start 111.3788 87.3) (end 112.8268 85.852) (width 0.5) (layer "F.Cu") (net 26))
 (segment (start 112.8312 85.7054) (end 112.8312 82.0364) (width 0.5) (layer "F.Cu") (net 26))
 (segment (start 115.0152 85.8464) (end 112.9722 85.8464) (width 0.5) (layer "F.Cu") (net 26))
 (segment (start 112.7252 95.3628) (end 112.7252 93.98) (width 0.5) (layer "F.Cu") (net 26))
 (segment (start 112.8312 82.0364) (end 112.0552 81.2604) (width 0.5) (layer "F.Cu") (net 26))
 (segment (start 112.9722 85.8464) (end 112.8312 85.7054) (width 0.5) (layer "F.Cu") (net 26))
 (via (at 112.7252 93.98) (size 0.8) (drill 0.5) (layers "F.Cu" "B.Cu") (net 26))
 (via (at 112.8268 85.852) (size 0.8) (drill 0.5) (layers "F.Cu" "B.Cu") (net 26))
 (segment (start 112.7252 85.9536) (end 112.8268 85.852) (width 0.5) (layer "B.Cu") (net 26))
 (segment (start 112.7252 93.98) (end 112.7252 85.9536) (width 0.5) (layer "B.Cu") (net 26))
 (segment (start 111.1108 95.3628) (end 110.8456 95.3628) (width 0.5) (layer "F.Cu") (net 27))
 (segment (start 112.5108 96.7628) (end 111.1108 95.3628) (width 0.5) (layer "F.Cu") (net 27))
 (segment (start 112.7252 96.7628) (end 112.5108 96.7628) (width 0.5) (layer "F.Cu") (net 27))
 (segment (start 123.4622 87.5082) (end 123.444 87.49) (width 0.3) (layer "F.Cu") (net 28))
 (segment (start 125.1027 87.5082) (end 123.4622 87.5082) (width 0.3) (layer "F.Cu") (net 28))
 (segment (start 109.9252 93.9604) (end 110.6052 93.2804) (width 0.5) (layer "F.Cu") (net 10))
 (segment (start 105.7852 93.9604) (end 105.1052 93.2804) (width 0.5) (layer "F.Cu") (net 10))
 (segment (start 109.6562 79.3554) (end 114.3552 79.3554) (width 0.5) (layer "F.Cu") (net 10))
 (segment (start 107.8992 92.9132) (end 106.5784 91.5924) (width 0.5) (layer "F.Cu") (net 10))
 (segment (start 122.428 100.4316) (end 122.1232 100.7364) (width 0.5) (layer "F.Cu") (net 10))
 (segment (start 122.2502 77.3938) (end 118.1862 77.3938) (width 0.5) (layer "F.Cu") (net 10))
 (segment (start 109.9252 83.8004) (end 110.6052 84.4804) (width 0.5) (layer "F.Cu") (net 10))
 (segment (start 102.9252 83.8004) (end 104.4252 83.8004) (width 0.5) (layer "F.Cu") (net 10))
 (segment (start 108.0052 93.9604) (end 109.9252 93.9604) (width 0.5) (layer "F.Cu") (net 10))
 (segment (start 124.4854 77.3938) (end 122.2502 77.3938) (width 0.5) (layer "F.Cu") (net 10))
 (segment (start 119.7864 100.1268) (end 119.1768 100.7364) (width 0.5) (layer "F.Cu") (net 10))
 (segment (start 102.9252 93.9604) (end 104.4252 93.9604) (width 0.5) (layer "F.Cu") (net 10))
 (segment (start 104.4252 93.9604) (end 105.1052 93.2804) (width 0.5) (layer "F.Cu") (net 10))
 (segment (start 110.6052 90.4804) (end 110.6052 93.2804) (width 0.5) (layer "F.Cu") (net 10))
 (segment (start 119.7864 100.1268) (end 119.7864 99.4356) (width 0.5) (layer "F.Cu") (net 10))
 (segment (start 116.6027 78.9744) (end 116.0062 78.9744) (width 0.5) (layer "F.Cu") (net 10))
 (segment (start 108.0052 83.8004) (end 105.7852 83.8004) (width 0.5) (layer "F.Cu") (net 10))
 (segment (start 124.7648 83.0072) (end 124.7648 82.7024) (width 0.5) (layer "F.Cu") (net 10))
 (segment (start 124.5108 77.4192) (end 124.4854 77.3938) (width 0.5) (layer "F.Cu") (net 10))
 (segment (start 133.4472 87.6496) (end 132.736 88.3608) (width 0.5) (layer "F.Cu") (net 10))
 (segment (start 104.4252 83.8004) (end 105.1052 84.4804) (width 0.5) (layer "F.Cu") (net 10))
 (segment (start 131.884717 88.3499) (end 131.693017 88.1582) (width 0.3) (layer "F.Cu") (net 10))
 (segment (start 114.3552 79.3554) (end 114.9902 79.9904) (width 0.5) (layer "F.Cu") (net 10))
 (segment (start 130.1496 77.4192) (end 124.5108 77.4192) (width 0.5) (layer "F.Cu") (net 10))
 (segment (start 132.2788 88.3499) (end 131.884717 88.3499) (width 0.3) (layer "F.Cu") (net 10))
 (segment (start 118.1608 77.4192) (end 118.1579 77.4192) (width 0.5) (layer "F.Cu") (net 10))
 (segment (start 118.1579 77.4192) (end 116.6027 78.9744) (width 0.5) (layer "F.Cu") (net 10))
 (segment (start 108.9302 81.2604) (end 108.9302 80.0814) (width 0.5) (layer "F.Cu") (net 10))
 (segment (start 113.1835 100.7364) (end 112.8776 100.4305) (width 0.5) (layer "F.Cu") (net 10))
 (segment (start 106.5784 86.3092) (end 107.8992 84.9884) (width 0.5) (layer "F.Cu") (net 10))
 (segment (start 133.4472 85.0856) (end 133.4472 87.6496) (width 0.5) (layer "F.Cu") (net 10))
 (segment (start 119.7864 99.4356) (end 119.7766 99.4356) (width 0.5) (layer "F.Cu") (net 10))
 (segment (start 132.736 88.3608) (end 132.519221 88.3608) (width 0.5) (layer "F.Cu") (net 10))
 (segment (start 112.2559 90.9707) (end 111.7852 90.5) (width 0.3) (layer "F.Cu") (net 10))
 (segment (start 130.8277 88.1582) (end 131.693017 88.1582) (width 0.3) (layer "F.Cu") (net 10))
 (segment (start 114.9902 79.9904) (end 114.9902 81.2214) (width 0.5) (layer "F.Cu") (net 10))
 (segment (start 106.5784 91.5924) (end 106.5784 86.3092) (width 0.5) (layer "F.Cu") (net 10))
 (segment (start 108.9302 80.0814) (end 109.6562 79.3554) (width 0.5) (layer "F.Cu") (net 10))
 (segment (start 132.508321 88.3499) (end 132.2788 88.3499) (width 0.5) (layer "F.Cu") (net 10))
 (segment (start 122.1232 80.0608) (end 122.1232 77.5208) (width 0.5) (layer "F.Cu") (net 10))
 (segment (start 112.6744 90.9707) (end 112.2559 90.9707) (width 0.3) (layer "F.Cu") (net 10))
 (segment (start 131.4704 83.1088) (end 133.4472 85.0856) (width 0.5) (layer "F.Cu") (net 10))
 (segment (start 118.1862 77.3938) (end 118.1608 77.4192) (width 0.5) (layer "F.Cu") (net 10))
 (segment (start 111.7852 90.5) (end 110.4992 90.5) (width 0.3) (layer "F.Cu") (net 10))
 (segment (start 107.8992 93.98) (end 107.8992 92.9132) (width 0.5) (layer "F.Cu") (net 10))
 (segment (start 122.1232 100.7364) (end 120.396 100.7364) (width 0.5) (layer "F.Cu") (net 10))
 (segment (start 107.8992 84.9884) (end 107.8992 83.82) (width 0.5) (layer "F.Cu") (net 10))
 (segment (start 108.0052 83.8004) (end 108.0052 82.1854) (width 0.5) (layer "F.Cu") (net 10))
 (segment (start 108.0052 83.8004) (end 109.9252 83.8004) (width 0.5) (layer "F.Cu") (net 10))
 (segment (start 108.0052 93.9604) (end 105.7852 93.9604) (width 0.5) (layer "F.Cu") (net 10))
 (segment (start 120.396 100.7364) (end 119.7864 100.1268) (width 0.5) (layer "F.Cu") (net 10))
 (segment (start 105.7852 83.8004) (end 105.1052 84.4804) (width 0.5) (layer "F.Cu") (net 10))
 (segment (start 108.0052 82.1854) (end 108.9302 81.2604) (width 0.5) (layer "F.Cu") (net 10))
 (segment (start 104.9992 93.3) (end 104.9992 84.5) (width 0.5) (layer "F.Cu") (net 10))
 (segment (start 119.1768 100.7364) (end 113.1835 100.7364) (width 0.5) (layer "F.Cu") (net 10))
 (segment (start 123.444 84.328) (end 124.7648 83.0072) (width 0.5) (layer "F.Cu") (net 10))
 (segment (start 124.7648 82.7024) (end 122.1232 80.0608) (width 0.5) (layer "F.Cu") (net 10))
 (segment (start 102.8192 93.98) (end 102.8192 83.82) (width 0.5) (layer "F.Cu") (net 10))
 (segment (start 114.9902 81.2214) (end 115.0152 81.2464) (width 0.5) (layer "F.Cu") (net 10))
 (segment (start 123.444 84.7765) (end 123.444 84.328) (width 0.5) (layer "F.Cu") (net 10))
 (segment (start 132.519221 88.3608) (end 132.508321 88.3499) (width 0.5) (layer "F.Cu") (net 10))
 (segment (start 122.428 99.1831) (end 122.428 100.4316) (width 0.5) (layer "F.Cu") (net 10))
 (segment (start 116.0062 78.9744) (end 114.9902 79.9904) (width 0.5) (layer "F.Cu") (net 10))
 (via (at 124.7648 83.0072) (size 1) (drill 0.5) (layers "F.Cu" "B.Cu") (free) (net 10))
 (via (at 131.3688 83.0072) (size 1) (drill 0.5) (layers "F.Cu" "B.Cu") (free) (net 10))
 (via (at 130.1496 77.4192) (size 1) (drill 0.5) (layers "F.Cu" "B.Cu") (free) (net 10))
 (via (at 124.4854 77.3938) (size 1) (drill 0.5) (layers "F.Cu" "B.Cu") (free) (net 10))
 (segment (start 123.6394 78.2398) (end 123.6394 81.8818) (width 0.5) (layer "B.Cu") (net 10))
 (segment (start 131.318 78.5876) (end 131.318 83.1088) (width 0.5) (layer "B.Cu") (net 10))
 (segment (start 123.6394 81.8818) (end 124.7648 83.0072) (width 0.5) (layer "B.Cu") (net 10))
 (segment (start 124.4854 77.3938) (end 123.6394 78.2398) (width 0.5) (layer "B.Cu") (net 10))
 (segment (start 130.1496 77.4192) (end 131.318 78.5876) (width 0.5) (layer "B.Cu") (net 10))
 (segment (start 145.2225 97.155) (end 141.605 97.155) (width 1) (layer "F.Cu") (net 56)))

